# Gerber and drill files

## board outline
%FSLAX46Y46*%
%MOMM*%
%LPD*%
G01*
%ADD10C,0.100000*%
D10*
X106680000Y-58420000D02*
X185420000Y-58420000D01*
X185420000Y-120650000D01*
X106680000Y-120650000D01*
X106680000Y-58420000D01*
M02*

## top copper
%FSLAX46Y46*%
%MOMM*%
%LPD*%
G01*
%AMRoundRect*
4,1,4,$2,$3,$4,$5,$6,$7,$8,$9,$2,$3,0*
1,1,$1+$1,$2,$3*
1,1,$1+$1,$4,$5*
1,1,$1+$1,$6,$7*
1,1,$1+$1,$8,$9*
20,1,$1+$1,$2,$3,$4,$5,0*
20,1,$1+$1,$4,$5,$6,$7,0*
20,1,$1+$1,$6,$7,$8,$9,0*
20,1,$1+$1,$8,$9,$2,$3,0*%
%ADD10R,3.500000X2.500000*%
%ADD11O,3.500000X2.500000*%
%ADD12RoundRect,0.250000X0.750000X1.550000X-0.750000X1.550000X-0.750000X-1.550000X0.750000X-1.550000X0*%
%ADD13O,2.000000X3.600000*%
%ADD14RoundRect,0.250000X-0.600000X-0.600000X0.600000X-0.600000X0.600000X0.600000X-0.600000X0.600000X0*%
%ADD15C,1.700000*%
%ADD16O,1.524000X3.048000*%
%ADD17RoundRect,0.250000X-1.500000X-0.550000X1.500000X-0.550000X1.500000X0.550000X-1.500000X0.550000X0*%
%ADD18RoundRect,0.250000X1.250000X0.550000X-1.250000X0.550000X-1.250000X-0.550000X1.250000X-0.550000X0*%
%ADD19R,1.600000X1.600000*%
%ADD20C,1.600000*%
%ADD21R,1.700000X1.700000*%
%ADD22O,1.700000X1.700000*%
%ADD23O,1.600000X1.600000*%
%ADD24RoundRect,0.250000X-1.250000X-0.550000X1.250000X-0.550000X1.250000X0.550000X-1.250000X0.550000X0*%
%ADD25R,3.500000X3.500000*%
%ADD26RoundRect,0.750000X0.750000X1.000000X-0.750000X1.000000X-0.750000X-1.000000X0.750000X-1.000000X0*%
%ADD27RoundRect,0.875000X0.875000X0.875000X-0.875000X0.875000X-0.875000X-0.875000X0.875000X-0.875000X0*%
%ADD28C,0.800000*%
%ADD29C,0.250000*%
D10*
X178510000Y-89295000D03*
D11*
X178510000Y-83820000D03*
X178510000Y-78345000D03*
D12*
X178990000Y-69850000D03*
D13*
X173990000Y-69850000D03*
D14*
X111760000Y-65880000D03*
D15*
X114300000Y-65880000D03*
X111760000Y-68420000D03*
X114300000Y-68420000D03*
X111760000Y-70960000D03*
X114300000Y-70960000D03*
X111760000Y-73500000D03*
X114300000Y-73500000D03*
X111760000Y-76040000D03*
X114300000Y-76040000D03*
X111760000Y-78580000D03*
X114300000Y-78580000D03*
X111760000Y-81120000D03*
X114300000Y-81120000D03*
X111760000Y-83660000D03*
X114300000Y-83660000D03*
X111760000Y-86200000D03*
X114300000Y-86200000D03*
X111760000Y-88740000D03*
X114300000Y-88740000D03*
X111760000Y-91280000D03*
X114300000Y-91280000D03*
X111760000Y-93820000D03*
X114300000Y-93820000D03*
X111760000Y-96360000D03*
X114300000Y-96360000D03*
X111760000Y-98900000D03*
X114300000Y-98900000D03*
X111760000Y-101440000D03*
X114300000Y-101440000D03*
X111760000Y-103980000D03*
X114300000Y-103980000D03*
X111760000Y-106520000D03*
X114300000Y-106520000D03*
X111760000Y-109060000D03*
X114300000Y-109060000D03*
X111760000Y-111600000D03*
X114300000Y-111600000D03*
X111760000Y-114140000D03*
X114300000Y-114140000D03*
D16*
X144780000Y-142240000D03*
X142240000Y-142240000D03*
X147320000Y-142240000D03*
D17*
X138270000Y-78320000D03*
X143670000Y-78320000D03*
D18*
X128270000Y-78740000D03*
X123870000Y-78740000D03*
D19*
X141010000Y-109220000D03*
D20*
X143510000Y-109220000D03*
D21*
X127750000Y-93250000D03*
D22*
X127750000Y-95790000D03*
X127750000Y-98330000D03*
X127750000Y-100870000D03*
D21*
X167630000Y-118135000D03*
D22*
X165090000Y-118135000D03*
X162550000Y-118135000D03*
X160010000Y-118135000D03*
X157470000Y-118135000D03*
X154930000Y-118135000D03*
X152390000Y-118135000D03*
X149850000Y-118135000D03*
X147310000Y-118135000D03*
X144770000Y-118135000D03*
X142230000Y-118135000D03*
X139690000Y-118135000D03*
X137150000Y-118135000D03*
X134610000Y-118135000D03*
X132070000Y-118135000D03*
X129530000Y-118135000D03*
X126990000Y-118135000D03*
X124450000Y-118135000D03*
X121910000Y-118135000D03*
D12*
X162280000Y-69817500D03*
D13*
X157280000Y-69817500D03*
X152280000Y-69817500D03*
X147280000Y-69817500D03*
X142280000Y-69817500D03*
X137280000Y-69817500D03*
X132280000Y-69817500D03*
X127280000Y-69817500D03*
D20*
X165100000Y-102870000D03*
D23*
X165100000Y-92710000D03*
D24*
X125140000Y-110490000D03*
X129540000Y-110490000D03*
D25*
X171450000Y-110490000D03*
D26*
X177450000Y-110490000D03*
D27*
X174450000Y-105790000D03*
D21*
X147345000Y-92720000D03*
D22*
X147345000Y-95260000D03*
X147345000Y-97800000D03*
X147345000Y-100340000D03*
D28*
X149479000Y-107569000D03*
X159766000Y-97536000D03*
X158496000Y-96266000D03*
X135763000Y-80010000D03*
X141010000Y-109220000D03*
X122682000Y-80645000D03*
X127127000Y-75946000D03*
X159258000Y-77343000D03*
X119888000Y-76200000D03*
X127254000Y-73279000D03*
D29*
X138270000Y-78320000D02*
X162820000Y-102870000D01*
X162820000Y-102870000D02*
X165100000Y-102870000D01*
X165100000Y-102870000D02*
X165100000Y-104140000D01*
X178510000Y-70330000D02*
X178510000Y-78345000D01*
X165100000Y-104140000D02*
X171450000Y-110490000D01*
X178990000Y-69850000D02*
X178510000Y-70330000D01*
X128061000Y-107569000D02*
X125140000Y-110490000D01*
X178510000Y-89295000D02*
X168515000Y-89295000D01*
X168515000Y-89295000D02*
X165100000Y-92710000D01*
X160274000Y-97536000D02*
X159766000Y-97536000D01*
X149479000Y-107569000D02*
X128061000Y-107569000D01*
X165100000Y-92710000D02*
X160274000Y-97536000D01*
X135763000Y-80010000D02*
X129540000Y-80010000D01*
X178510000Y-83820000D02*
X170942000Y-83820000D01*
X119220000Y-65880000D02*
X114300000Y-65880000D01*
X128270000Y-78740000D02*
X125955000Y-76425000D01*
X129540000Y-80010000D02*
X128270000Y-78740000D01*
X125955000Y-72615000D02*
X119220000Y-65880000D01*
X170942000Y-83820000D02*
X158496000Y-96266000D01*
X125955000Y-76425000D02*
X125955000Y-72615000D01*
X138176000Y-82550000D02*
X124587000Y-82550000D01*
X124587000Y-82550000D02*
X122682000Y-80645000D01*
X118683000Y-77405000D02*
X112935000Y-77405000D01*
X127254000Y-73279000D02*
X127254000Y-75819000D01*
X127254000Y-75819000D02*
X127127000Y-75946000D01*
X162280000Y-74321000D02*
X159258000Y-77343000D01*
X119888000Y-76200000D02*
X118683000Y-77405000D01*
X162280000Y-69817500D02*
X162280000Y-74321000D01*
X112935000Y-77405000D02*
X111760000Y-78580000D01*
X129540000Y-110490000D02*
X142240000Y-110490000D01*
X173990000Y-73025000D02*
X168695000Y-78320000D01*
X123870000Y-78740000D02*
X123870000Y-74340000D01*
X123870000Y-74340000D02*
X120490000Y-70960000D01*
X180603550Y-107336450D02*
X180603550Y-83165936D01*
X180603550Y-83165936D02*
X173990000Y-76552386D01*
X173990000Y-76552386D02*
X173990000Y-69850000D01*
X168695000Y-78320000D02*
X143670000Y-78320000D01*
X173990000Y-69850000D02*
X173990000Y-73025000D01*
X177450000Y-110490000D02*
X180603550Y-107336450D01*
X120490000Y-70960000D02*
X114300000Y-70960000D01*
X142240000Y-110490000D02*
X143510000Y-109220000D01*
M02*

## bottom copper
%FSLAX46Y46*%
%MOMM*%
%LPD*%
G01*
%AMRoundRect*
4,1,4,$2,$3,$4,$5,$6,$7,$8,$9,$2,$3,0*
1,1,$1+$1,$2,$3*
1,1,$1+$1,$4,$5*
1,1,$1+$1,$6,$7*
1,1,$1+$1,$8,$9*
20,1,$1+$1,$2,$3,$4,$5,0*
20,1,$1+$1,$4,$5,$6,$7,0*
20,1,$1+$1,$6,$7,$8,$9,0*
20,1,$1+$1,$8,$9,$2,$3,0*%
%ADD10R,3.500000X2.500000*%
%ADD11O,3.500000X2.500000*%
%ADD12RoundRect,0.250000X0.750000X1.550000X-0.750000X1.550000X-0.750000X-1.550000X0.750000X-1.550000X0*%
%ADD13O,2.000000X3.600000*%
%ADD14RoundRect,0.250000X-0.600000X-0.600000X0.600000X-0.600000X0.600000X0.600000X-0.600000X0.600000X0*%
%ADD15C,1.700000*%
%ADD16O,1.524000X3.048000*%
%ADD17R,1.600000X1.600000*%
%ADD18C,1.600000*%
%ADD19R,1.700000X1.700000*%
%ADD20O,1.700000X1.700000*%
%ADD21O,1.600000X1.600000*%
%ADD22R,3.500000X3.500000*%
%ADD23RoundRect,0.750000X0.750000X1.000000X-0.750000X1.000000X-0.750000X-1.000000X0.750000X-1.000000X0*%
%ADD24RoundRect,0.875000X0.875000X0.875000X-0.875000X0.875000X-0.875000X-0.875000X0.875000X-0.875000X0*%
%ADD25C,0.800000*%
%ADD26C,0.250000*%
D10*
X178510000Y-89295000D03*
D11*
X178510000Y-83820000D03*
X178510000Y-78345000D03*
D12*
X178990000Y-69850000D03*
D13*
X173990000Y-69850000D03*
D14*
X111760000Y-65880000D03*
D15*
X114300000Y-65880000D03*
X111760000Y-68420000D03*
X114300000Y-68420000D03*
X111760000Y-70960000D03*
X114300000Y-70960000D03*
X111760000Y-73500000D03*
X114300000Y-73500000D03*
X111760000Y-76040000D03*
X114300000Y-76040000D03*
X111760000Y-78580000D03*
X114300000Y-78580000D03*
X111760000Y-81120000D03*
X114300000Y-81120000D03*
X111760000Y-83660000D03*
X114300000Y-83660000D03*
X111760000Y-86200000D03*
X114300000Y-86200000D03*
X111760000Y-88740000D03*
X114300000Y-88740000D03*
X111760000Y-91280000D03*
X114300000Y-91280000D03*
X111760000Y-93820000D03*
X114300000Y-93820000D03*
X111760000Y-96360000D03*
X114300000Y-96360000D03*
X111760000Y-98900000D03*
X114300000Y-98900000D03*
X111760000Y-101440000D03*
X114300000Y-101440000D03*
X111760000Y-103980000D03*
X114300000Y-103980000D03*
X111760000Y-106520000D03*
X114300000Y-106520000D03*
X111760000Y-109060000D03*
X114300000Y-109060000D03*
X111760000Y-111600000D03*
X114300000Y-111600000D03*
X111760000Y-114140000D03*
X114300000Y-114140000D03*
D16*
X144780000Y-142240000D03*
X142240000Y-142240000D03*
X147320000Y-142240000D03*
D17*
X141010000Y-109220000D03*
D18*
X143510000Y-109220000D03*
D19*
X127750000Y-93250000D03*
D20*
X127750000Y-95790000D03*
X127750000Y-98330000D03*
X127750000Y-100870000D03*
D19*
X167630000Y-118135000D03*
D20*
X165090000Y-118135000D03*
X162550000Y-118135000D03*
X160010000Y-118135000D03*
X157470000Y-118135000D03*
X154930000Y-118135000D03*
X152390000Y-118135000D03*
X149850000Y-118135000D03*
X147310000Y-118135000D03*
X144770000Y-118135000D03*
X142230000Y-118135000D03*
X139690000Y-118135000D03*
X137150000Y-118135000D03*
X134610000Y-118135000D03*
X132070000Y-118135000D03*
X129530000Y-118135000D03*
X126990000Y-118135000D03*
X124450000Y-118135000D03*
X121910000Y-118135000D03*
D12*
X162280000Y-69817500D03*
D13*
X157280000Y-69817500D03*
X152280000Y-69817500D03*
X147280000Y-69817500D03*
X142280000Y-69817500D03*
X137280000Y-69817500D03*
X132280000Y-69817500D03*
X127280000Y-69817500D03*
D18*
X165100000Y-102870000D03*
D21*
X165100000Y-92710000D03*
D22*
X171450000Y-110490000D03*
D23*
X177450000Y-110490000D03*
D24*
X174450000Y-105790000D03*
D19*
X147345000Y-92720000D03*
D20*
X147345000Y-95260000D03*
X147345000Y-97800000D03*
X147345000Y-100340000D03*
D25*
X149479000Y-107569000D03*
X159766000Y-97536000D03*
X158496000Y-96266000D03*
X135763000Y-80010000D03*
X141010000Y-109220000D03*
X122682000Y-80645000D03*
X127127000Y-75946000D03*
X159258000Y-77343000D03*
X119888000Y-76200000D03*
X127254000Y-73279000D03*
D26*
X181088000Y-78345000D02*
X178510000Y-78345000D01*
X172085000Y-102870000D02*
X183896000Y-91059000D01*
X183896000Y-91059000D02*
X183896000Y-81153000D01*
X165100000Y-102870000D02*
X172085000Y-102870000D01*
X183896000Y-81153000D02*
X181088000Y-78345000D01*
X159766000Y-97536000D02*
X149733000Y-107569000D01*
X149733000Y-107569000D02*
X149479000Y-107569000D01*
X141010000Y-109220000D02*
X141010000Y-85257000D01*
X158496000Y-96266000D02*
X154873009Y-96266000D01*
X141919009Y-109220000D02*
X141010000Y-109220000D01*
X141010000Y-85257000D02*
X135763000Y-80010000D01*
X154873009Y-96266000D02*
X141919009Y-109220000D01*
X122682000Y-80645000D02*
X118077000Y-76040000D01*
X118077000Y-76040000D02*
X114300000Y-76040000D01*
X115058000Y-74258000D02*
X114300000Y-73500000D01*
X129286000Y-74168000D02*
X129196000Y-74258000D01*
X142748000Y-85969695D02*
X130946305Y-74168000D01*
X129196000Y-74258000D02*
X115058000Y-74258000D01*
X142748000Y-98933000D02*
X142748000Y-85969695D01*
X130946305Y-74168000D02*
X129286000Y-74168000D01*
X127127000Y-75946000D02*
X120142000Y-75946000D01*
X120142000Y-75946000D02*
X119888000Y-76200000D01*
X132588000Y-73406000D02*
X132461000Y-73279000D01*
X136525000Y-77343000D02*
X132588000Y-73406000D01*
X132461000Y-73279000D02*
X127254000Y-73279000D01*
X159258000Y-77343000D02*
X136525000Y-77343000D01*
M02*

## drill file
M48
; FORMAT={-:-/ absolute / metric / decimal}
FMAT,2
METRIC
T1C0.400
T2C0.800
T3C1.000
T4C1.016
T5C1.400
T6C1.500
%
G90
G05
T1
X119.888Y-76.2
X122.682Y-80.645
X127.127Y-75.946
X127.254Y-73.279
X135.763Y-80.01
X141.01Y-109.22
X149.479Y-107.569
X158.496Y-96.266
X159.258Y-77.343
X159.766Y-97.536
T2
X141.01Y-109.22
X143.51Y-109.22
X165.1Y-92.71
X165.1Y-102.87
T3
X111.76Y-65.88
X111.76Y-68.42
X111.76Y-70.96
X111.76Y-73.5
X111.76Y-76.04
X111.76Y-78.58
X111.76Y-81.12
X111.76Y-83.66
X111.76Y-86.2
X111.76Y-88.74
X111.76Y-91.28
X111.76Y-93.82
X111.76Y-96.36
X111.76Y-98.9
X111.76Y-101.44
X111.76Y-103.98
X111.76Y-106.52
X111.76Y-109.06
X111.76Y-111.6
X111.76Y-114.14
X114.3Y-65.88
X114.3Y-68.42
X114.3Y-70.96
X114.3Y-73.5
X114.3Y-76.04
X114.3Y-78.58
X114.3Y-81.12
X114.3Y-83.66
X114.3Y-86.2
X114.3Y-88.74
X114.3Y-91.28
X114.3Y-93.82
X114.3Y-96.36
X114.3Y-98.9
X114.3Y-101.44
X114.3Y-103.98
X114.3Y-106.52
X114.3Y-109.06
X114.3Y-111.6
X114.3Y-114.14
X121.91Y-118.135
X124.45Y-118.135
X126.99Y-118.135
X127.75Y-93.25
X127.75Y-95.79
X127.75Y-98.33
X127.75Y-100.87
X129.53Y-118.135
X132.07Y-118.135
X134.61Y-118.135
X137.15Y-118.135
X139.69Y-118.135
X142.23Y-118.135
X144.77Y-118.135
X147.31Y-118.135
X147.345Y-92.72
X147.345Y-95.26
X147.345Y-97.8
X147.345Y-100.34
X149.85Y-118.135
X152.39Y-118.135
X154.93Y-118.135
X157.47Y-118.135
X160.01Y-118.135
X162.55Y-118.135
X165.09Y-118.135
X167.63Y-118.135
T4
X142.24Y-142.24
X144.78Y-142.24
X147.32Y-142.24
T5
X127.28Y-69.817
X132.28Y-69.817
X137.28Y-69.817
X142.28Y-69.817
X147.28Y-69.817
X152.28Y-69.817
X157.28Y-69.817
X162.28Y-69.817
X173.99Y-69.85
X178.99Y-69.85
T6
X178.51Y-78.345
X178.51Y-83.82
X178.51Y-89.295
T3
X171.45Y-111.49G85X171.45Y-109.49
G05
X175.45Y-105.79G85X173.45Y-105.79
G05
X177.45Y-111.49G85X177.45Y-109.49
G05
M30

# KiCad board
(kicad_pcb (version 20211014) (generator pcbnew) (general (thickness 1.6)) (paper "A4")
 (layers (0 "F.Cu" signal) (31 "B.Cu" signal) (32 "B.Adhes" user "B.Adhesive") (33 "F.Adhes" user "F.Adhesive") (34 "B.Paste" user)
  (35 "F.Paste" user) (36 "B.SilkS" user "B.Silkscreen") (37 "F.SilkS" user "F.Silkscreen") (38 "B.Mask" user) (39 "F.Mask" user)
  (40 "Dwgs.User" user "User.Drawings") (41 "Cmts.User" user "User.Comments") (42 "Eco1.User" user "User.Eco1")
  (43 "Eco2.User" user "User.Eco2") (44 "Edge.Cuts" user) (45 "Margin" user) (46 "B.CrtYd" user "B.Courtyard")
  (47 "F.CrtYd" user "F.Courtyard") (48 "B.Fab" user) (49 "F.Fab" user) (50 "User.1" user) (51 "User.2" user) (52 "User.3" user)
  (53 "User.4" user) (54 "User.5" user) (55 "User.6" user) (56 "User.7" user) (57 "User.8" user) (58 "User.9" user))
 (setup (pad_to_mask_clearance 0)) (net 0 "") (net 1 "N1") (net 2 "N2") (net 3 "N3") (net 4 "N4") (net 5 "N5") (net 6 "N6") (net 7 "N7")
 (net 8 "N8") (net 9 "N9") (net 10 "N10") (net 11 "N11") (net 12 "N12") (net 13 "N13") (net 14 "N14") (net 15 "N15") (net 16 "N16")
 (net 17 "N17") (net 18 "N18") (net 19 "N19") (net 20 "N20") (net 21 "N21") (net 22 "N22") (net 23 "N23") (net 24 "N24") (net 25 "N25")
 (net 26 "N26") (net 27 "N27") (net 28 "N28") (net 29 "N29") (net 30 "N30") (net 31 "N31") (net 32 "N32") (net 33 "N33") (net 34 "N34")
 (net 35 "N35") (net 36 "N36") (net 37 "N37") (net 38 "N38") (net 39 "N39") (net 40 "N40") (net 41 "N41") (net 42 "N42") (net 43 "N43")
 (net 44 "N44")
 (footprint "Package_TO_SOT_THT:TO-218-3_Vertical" (layer "F.Cu") (at 178.51 89.295 90)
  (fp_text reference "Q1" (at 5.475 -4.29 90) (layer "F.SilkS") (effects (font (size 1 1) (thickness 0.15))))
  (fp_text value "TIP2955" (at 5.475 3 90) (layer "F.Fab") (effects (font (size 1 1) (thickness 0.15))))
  (pad "1" thru_hole rect (at 0 0 90) (size 2.5 3.5) (drill 1.5) (layers *.Cu *.Mask) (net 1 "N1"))
  (pad "2" thru_hole oval (at 5.475 0 90) (size 2.5 3.5) (drill 1.5) (layers *.Cu *.Mask) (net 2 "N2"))
  (pad "3" thru_hole oval (at 10.95 0 90) (size 2.5 3.5) (drill 1.5) (layers *.Cu *.Mask) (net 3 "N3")))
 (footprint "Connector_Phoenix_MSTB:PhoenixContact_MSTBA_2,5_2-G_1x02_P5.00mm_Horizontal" (layer "F.Cu") (at 178.99 69.85 180)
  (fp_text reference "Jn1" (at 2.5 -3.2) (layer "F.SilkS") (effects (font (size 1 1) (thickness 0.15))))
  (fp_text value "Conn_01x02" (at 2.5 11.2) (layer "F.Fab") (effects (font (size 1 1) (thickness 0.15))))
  (pad "1" thru_hole roundrect (at 0 0 180) (size 2 3.6) (drill 1.4) (layers *.Cu *.Mask) (roundrect_rratio 0.125) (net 3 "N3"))
  (pad "2" thru_hole oval (at 5 0 180) (size 2 3.6) (drill 1.4) (layers *.Cu *.Mask) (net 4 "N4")))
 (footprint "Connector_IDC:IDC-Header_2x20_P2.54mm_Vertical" (layer "F.Cu") (at 111.76 65.88)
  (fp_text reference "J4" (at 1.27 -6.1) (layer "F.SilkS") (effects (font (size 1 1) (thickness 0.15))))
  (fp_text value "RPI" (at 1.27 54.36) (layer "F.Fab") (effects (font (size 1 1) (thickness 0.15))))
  (pad "1" thru_hole roundrect (at 0 0) (size 1.7 1.7) (drill 1) (layers *.Cu *.Mask) (roundrect_rratio 0.147059) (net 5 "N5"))
  (pad "2" thru_hole circle (at 2.54 0) (size 1.7 1.7) (drill 1) (layers *.Cu *.Mask) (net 2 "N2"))
  (pad "3" thru_hole circle (at 0 2.54) (size 1.7 1.7) (drill 1) (layers *.Cu *.Mask) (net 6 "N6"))
  (pad "4" thru_hole circle (at 2.54 2.54) (size 1.7 1.7) (drill 1) (layers *.Cu *.Mask) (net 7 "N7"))
  (pad "5" thru_hole circle (at 0 5.08) (size 1.7 1.7) (drill 1) (layers *.Cu *.Mask) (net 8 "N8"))
  (pad "6" thru_hole circle (at 2.54 5.08) (size 1.7 1.7) (drill 1) (layers *.Cu *.Mask) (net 4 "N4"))
  (pad "7" thru_hole circle (at 0 7.62) (size 1.7 1.7) (drill 1) (layers *.Cu *.Mask) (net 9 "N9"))
  (pad "8" thru_hole circle (at 2.54 7.62) (size 1.7 1.7) (drill 1) (layers *.Cu *.Mask) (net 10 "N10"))
  (pad "9" thru_hole circle (at 0 10.16) (size 1.7 1.7) (drill 1) (layers *.Cu *.Mask) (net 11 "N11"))
  (pad "10" thru_hole circle (at 2.54 10.16) (size 1.7 1.7) (drill 1) (layers *.Cu *.Mask) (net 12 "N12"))
  (pad "11" thru_hole circle (at 0 12.7) (size 1.7 1.7) (drill 1) (layers *.Cu *.Mask) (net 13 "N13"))
  (pad "12" thru_hole circle (at 2.54 12.7) (size 1.7 1.7) (drill 1) (layers *.Cu *.Mask) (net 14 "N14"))
  (pad "13" thru_hole circle (at 0 15.24) (size 1.7 1.7) (drill 1) (layers *.Cu *.Mask) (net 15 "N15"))
  (pad "14" thru_hole circle (at 2.54 15.24) (size 1.7 1.7) (drill 1) (layers *.Cu *.Mask) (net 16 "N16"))
  (pad "15" thru_hole circle (at 0 17.78) (size 1.7 1.7) (drill 1) (layers *.Cu *.Mask) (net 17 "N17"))
  (pad "16" thru_hole circle (at 2.54 17.78) (size 1.7 1.7) (drill 1) (layers *.Cu *.Mask) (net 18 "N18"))
  (pad "17" thru_hole circle (at 0 20.32) (size 1.7 1.7) (drill 1) (layers *.Cu *.Mask) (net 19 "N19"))
  (pad "18" thru_hole circle (at 2.54 20.32) (size 1.7 1.7) (drill 1) (layers *.Cu *.Mask) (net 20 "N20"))
  (pad "19" thru_hole circle (at 0 22.86) (size 1.7 1.7) (drill 1) (layers *.Cu *.Mask) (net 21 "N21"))
  (pad "20" thru_hole circle (at 2.54 22.86) (size 1.7 1.7) (drill 1) (layers *.Cu *.Mask) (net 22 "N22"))
  (pad "21" thru_hole circle (at 0 25.4) (size 1.7 1.7) (drill 1) (layers *.Cu *.Mask) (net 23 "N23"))
  (pad "22" thru_hole circle (at 2.54 25.4) (size 1.7 1.7) (drill 1) (layers *.Cu *.Mask) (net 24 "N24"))
  (pad "23" thru_hole circle (at 0 27.94) (size 1.7 1.7) (drill 1) (layers *.Cu *.Mask) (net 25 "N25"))
  (pad "24" thru_hole circle (at 2.54 27.94) (size 1.7 1.7) (drill 1) (layers *.Cu *.Mask) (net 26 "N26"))
  (pad "25" thru_hole circle (at 0 30.48) (size 1.7 1.7) (drill 1) (layers *.Cu *.Mask) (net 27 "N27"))
  (pad "26" thru_hole circle (at 2.54 30.48) (size 1.7 1.7) (drill 1) (layers *.Cu *.Mask) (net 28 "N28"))
  (pad "27" thru_hole circle (at 0 33.02) (size 1.7 1.7) (drill 1) (layers *.Cu *.Mask) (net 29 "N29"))
  (pad "28" thru_hole circle (at 2.54 33.02) (size 1.7 1.7) (drill 1) (layers *.Cu *.Mask) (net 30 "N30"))
  (pad "29" thru_hole circle (at 0 35.56) (size 1.7 1.7) (drill 1) (layers *.Cu *.Mask) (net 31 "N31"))
  (pad "30" thru_hole circle (at 2.54 35.56) (size 1.7 1.7) (drill 1) (layers *.Cu *.Mask) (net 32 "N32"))
  (pad "31" thru_hole circle (at 0 38.1) (size 1.7 1.7) (drill 1) (layers *.Cu *.Mask) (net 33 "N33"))
  (pad "32" thru_hole circle (at 2.54 38.1) (size 1.7 1.7) (drill 1) (layers *.Cu *.Mask) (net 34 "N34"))
  (pad "33" thru_hole circle (at 0 40.64) (size 1.7 1.7) (drill 1) (layers *.Cu *.Mask) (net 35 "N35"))
  (pad "34" thru_hole circle (at 2.54 40.64) (size 1.7 1.7) (drill 1) (layers *.Cu *.Mask) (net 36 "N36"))
  (pad "35" thru_hole circle (at 0 43.18) (size 1.7 1.7) (drill 1) (layers *.Cu *.Mask) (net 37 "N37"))
  (pad "36" thru_hole circle (at 2.54 43.18) (size 1.7 1.7) (drill 1) (layers *.Cu *.Mask) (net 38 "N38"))
  (pad "37" thru_hole circle (at 0 45.72) (size 1.7 1.7) (drill 1) (layers *.Cu *.Mask) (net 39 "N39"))
  (pad "38" thru_hole circle (at 2.54 45.72) (size 1.7 1.7) (drill 1) (layers *.Cu *.Mask) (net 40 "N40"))
  (pad "39" thru_hole circle (at 0 48.26) (size 1.7 1.7) (drill 1) (layers *.Cu *.Mask) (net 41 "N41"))
  (pad "40" thru_hole circle (at 2.54 48.26) (size 1.7 1.7) (drill 1) (layers *.Cu *.Mask) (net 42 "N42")))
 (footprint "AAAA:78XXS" (layer "F.Cu") (at 144.78 139.7)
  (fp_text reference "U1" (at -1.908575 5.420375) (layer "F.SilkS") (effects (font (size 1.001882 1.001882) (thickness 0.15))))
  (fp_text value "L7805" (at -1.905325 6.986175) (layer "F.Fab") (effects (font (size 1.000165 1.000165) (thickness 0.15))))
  (pad "GND" thru_hole oval locked (at 0 2.54) (size 1.524 3.048) (drill 1.016) (layers *.Cu *.Mask))
  (pad "IN" thru_hole oval locked (at -2.54 2.54) (size 1.524 3.048) (drill 1.016) (layers *.Cu *.Mask))
  (pad "OUT" thru_hole oval locked (at 2.54 2.54) (size 1.524 3.048) (drill 1.016) (layers *.Cu *.Mask)))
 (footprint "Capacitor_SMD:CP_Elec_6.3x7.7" (layer "F.Cu") (at 140.97 78.32)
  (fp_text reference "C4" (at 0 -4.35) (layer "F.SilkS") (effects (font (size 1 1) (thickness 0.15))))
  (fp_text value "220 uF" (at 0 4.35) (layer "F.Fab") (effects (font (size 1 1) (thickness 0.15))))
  (pad "1" smd roundrect (at -2.7 0) (size 3.5 1.6) (layers "F.Cu" "F.Paste" "F.Mask") (roundrect_rratio 0.15625) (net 3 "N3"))
  (pad "2" smd roundrect (at 2.7 0) (size 3.5 1.6) (layers "F.Cu" "F.Paste" "F.Mask") (roundrect_rratio 0.15625) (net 4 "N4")))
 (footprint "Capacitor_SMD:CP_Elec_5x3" (layer "F.Cu") (at 126.07 78.74 180)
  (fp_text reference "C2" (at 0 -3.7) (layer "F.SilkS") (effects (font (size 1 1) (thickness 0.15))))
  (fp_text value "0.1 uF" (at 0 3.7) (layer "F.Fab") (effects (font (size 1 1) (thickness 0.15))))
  (pad "1" smd roundrect (at -2.2 0 180) (size 3 1.6) (layers "F.Cu" "F.Paste" "F.Mask") (roundrect_rratio 0.15625) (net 2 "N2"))
  (pad "2" smd roundrect (at 2.2 0 180) (size 3 1.6) (layers "F.Cu" "F.Paste" "F.Mask") (roundrect_rratio 0.15625) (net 4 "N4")))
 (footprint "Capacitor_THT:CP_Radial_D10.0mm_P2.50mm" (layer "F.Cu") (at 141.01 109.22)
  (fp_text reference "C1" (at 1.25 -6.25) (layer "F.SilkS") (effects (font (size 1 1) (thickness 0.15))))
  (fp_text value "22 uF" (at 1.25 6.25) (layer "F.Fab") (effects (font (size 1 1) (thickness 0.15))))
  (pad "1" thru_hole rect (at 0 0) (size 1.6 1.6) (drill 0.8) (layers *.Cu *.Mask) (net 2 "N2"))
  (pad "2" thru_hole circle (at 2.5 0) (size 1.6 1.6) (drill 0.8) (layers *.Cu *.Mask) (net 4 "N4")))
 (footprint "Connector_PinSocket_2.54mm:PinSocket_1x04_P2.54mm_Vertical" (layer "F.Cu") (at 127.75 93.25)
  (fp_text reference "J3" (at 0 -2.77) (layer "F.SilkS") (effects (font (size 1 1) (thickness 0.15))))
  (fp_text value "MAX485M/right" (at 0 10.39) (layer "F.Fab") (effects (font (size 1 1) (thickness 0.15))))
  (pad "1" thru_hole rect (at 0 0) (size 1.7 1.7) (drill 1) (layers *.Cu *.Mask) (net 7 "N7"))
  (pad "2" thru_hole oval (at 0 2.54) (size 1.7 1.7) (drill 1) (layers *.Cu *.Mask) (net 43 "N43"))
  (pad "3" thru_hole oval (at 0 5.08) (size 1.7 1.7) (drill 1) (layers *.Cu *.Mask) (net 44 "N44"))
  (pad "4" thru_hole oval (at 0 7.62) (size 1.7 1.7) (drill 1) (layers *.Cu *.Mask) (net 16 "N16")))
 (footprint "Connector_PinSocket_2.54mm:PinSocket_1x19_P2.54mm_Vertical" (layer "F.Cu") (at 167.63 118.135 -90)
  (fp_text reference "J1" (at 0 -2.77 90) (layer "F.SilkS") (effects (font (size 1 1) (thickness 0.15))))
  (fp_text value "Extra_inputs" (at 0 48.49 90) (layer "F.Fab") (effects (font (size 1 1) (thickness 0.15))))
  (pad "1" thru_hole rect (at 0 0 270) (size 1.7 1.7) (drill 1) (layers *.Cu *.Mask) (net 5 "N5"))
  (pad "2" thru_hole oval (at 0 2.54 270) (size 1.7 1.7) (drill 1) (layers *.Cu *.Mask) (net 11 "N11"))
  (pad "3" thru_hole oval (at 0 5.08 270) (size 1.7 1.7) (drill 1) (layers *.Cu *.Mask) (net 19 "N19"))
  (pad "4" thru_hole oval (at 0 7.62 270) (size 1.7 1.7) (drill 1) (layers *.Cu *.Mask) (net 27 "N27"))
  (pad "5" thru_hole oval (at 0 10.16 270) (size 1.7 1.7) (drill 1) (layers *.Cu *.Mask) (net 6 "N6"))
  (pad "6" thru_hole oval (at 0 12.7 270) (size 1.7 1.7) (drill 1) (layers *.Cu *.Mask) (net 8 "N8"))
  (pad "7" thru_hole oval (at 0 15.24 270) (size 1.7 1.7) (drill 1) (layers *.Cu *.Mask) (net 9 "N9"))
  (pad "8" thru_hole oval (at 0 17.78 270) (size 1.7 1.7) (drill 1) (layers *.Cu *.Mask) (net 23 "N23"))
  (pad "9" thru_hole oval (at 0 20.32 270) (size 1.7 1.7) (drill 1) (layers *.Cu *.Mask) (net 21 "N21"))
  (pad "10" thru_hole oval (at 0 22.86 270) (size 1.7 1.7) (drill 1) (layers *.Cu *.Mask) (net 25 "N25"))
  (pad "11" thru_hole oval (at 0 25.4 270) (size 1.7 1.7) (drill 1) (layers *.Cu *.Mask) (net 35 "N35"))
  (pad "12" thru_hole oval (at 0 27.94 270) (size 1.7 1.7) (drill 1) (layers *.Cu *.Mask) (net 37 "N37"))
  (pad "13" thru_hole oval (at 0 30.48 270) (size 1.7 1.7) (drill 1) (layers *.Cu *.Mask) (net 14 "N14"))
  (pad "14" thru_hole oval (at 0 33.02 270) (size 1.7 1.7) (drill 1) (layers *.Cu *.Mask) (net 24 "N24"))
  (pad "15" thru_hole oval (at 0 35.56 270) (size 1.7 1.7) (drill 1) (layers *.Cu *.Mask) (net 26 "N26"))
  (pad "16" thru_hole oval (at 0 38.1 270) (size 1.7 1.7) (drill 1) (layers *.Cu *.Mask) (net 28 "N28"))
  (pad "17" thru_hole oval (at 0 40.64 270) (size 1.7 1.7) (drill 1) (layers *.Cu *.Mask) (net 38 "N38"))
  (pad "18" thru_hole oval (at 0 43.18 270) (size 1.7 1.7) (drill 1) (layers *.Cu *.Mask) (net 40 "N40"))
  (pad "19" thru_hole oval (at 0 45.72 270) (size 1.7 1.7) (drill 1) (layers *.Cu *.Mask) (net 42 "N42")))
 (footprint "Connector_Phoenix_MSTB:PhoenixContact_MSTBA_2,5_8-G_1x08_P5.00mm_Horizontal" (layer "F.Cu") (at 162.28 69.8175 180)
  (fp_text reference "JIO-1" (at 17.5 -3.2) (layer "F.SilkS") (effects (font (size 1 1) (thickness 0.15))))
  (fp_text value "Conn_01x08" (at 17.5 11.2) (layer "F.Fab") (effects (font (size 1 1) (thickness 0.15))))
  (pad "1" thru_hole roundrect (at 0 0 180) (size 2 3.6) (drill 1.4) (layers *.Cu *.Mask) (roundrect_rratio 0.125) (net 13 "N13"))
  (pad "2" thru_hole oval (at 5 0 180) (size 2 3.6) (drill 1.4) (layers *.Cu *.Mask) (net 15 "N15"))
  (pad "3" thru_hole oval (at 10 0 180) (size 2 3.6) (drill 1.4) (layers *.Cu *.Mask) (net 17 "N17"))
  (pad "4" thru_hole oval (at 15 0 180) (size 2 3.6) (drill 1.4) (layers *.Cu *.Mask) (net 31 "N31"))
  (pad "5" thru_hole oval (at 20 0 180) (size 2 3.6) (drill 1.4) (layers *.Cu *.Mask) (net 33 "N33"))
  (pad "6" thru_hole oval (at 25 0 180) (size 2 3.6) (drill 1.4) (layers *.Cu *.Mask) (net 39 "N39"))
  (pad "7" thru_hole oval (at 30 0 180) (size 2 3.6) (drill 1.4) (layers *.Cu *.Mask) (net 18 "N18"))
  (pad "8" thru_hole oval (at 35 0 180) (size 2 3.6) (drill 1.4) (layers *.Cu *.Mask) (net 20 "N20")))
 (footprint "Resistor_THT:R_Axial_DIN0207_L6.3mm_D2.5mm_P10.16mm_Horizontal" (layer "F.Cu") (at 165.1 102.87 90)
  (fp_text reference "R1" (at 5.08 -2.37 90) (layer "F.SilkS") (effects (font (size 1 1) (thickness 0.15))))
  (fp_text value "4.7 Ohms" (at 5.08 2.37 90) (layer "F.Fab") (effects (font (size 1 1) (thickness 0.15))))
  (pad "1" thru_hole circle (at 0 0 90) (size 1.6 1.6) (drill 0.8) (layers *.Cu *.Mask) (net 3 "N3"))
  (pad "2" thru_hole oval (at 10.16 0 90) (size 1.6 1.6) (drill 0.8) (layers *.Cu *.Mask) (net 1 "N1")))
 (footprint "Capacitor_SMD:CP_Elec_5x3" (layer "F.Cu") (at 127.34 110.49)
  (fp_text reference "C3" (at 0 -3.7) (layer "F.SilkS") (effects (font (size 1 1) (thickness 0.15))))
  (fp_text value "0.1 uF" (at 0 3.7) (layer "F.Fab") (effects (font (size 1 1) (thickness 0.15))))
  (pad "1" smd roundrect (at -2.2 0) (size 3 1.6) (layers "F.Cu" "F.Paste" "F.Mask") (roundrect_rratio 0.15625) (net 1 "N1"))
  (pad "2" smd roundrect (at 2.2 0) (size 3 1.6) (layers "F.Cu" "F.Paste" "F.Mask") (roundrect_rratio 0.15625) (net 4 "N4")))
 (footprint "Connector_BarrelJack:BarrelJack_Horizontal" (layer "F.Cu") (at 171.45 110.49 180)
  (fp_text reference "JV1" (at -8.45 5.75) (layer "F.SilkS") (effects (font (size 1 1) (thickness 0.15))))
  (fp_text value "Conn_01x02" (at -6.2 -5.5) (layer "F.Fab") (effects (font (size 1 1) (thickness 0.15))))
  (pad "1" thru_hole rect (at 0 0 180) (size 3.5 3.5) (drill oval 1 3) (layers *.Cu *.Mask) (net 3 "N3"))
  (pad "2" thru_hole roundrect (at -6 0 180) (size 3 3.5) (drill oval 1 3) (layers *.Cu *.Mask) (roundrect_rratio 0.25) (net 4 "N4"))
  (pad "3" thru_hole roundrect (at -3 4.7 180) (size 3.5 3.5) (drill oval 3 1) (layers *.Cu *.Mask) (roundrect_rratio 0.25)))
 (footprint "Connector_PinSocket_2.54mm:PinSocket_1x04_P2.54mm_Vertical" (layer "F.Cu") (at 147.345 92.72)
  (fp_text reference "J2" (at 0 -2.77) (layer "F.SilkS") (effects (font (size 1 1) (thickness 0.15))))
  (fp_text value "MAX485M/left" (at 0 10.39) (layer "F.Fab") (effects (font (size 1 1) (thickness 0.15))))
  (pad "1" thru_hole rect (at 0 0) (size 1.7 1.7) (drill 1) (layers *.Cu *.Mask) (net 12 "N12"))
  (pad "2" thru_hole oval (at 0 2.54) (size 1.7 1.7) (drill 1) (layers *.Cu *.Mask) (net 34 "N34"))
  (pad "3" thru_hole oval (at 0 5.08) (size 1.7 1.7) (drill 1) (layers *.Cu *.Mask) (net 34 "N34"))
  (pad "4" thru_hole oval (at 0 7.62) (size 1.7 1.7) (drill 1) (layers *.Cu *.Mask) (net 10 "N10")))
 (gr_rect (start 106.68 120.65) (end 185.42 58.42) (layer "Edge.Cuts") (width 0.1) (fill none))
 (segment (start 138.27 78.32) (end 162.82 102.87) (width 0.25) (layer "F.Cu") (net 3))
 (segment (start 162.82 102.87) (end 165.1 102.87) (width 0.25) (layer "F.Cu") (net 3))
 (segment (start 165.1 102.87) (end 165.1 104.14) (width 0.25) (layer "F.Cu") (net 3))
 (segment (start 178.51 70.33) (end 178.51 78.345) (width 0.25) (layer "F.Cu") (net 3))
 (segment (start 165.1 104.14) (end 171.45 110.49) (width 0.25) (layer "F.Cu") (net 3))
 (segment (start 178.99 69.85) (end 178.51 70.33) (width 0.25) (layer "F.Cu") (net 3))
 (segment (start 181.088 78.345) (end 178.51 78.345) (width 0.25) (layer "B.Cu") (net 3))
 (segment (start 172.085 102.87) (end 183.896 91.059) (width 0.25) (layer "B.Cu") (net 3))
 (segment (start 183.896 91.059) (end 183.896 81.153) (width 0.25) (layer "B.Cu") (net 3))
 (segment (start 165.1 102.87) (end 172.085 102.87) (width 0.25) (layer "B.Cu") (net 3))
 (segment (start 183.896 81.153) (end 181.088 78.345) (width 0.25) (layer "B.Cu") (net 3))
 (segment (start 128.061 107.569) (end 125.14 110.49) (width 0.25) (layer "F.Cu") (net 1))
 (segment (start 178.51 89.295) (end 168.515 89.295) (width 0.25) (layer "F.Cu") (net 1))
 (segment (start 168.515 89.295) (end 165.1 92.71) (width 0.25) (layer "F.Cu") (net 1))
 (segment (start 160.274 97.536) (end 159.766 97.536) (width 0.25) (layer "F.Cu") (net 1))
 (segment (start 149.479 107.569) (end 128.061 107.569) (width 0.25) (layer "F.Cu") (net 1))
 (segment (start 165.1 92.71) (end 160.274 97.536) (width 0.25) (layer "F.Cu") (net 1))
 (via (at 149.479 107.569) (size 0.8) (drill 0.4) (layers "F.Cu" "B.Cu") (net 1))
 (via (at 159.766 97.536) (size 0.8) (drill 0.4) (layers "F.Cu" "B.Cu") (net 1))
 (segment (start 159.766 97.536) (end 149.733 107.569) (width 0.25) (layer "B.Cu") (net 1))
 (segment (start 149.733 107.569) (end 149.479 107.569) (width 0.25) (layer "B.Cu") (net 1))
 (segment (start 135.763 80.01) (end 129.54 80.01) (width 0.25) (layer "F.Cu") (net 2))
 (segment (start 178.51 83.82) (end 170.942 83.82) (width 0.25) (layer "F.Cu") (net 2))
 (segment (start 119.22 65.88) (end 114.3 65.88) (width 0.25) (layer "F.Cu") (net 2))
 (segment (start 128.27 78.74) (end 125.955 76.425) (width 0.25) (layer "F.Cu") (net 2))
 (segment (start 129.54 80.01) (end 128.27 78.74) (width 0.25) (layer "F.Cu") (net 2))
 (segment (start 125.955 72.615) (end 119.22 65.88) (width 0.25) (layer "F.Cu") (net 2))
 (segment (start 170.942 83.82) (end 158.496 96.266) (width 0.25) (layer "F.Cu") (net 2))
 (segment (start 125.955 76.425) (end 125.955 72.615) (width 0.25) (layer "F.Cu") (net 2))
 (via (at 158.496 96.266) (size 0.8) (drill 0.4) (layers "F.Cu" "B.Cu") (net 2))
 (via (at 135.763 80.01) (size 0.8) (drill 0.4) (layers "F.Cu" "B.Cu") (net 2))
 (via (at 141.01 109.22) (size 0.8) (drill 0.4) (layers "F.Cu" "B.Cu") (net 2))
 (segment (start 141.01 109.22) (end 141.01 85.257) (width 0.25) (layer "B.Cu") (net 2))
 (segment (start 158.496 96.266) (end 154.873009 96.266) (width 0.25) (layer "B.Cu") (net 2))
 (segment (start 141.919009 109.22) (end 141.01 109.22) (width 0.25) (layer "B.Cu") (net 2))
 (segment (start 141.01 85.257) (end 135.763 80.01) (width 0.25) (layer "B.Cu") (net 2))
 (segment (start 154.873009 96.266) (end 141.919009 109.22) (width 0.25) (layer "B.Cu") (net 2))
 (segment (start 138.176 82.55) (end 124.587 82.55) (width 0.25) (layer "F.Cu") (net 12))
 (segment (start 124.587 82.55) (end 122.682 80.645) (width 0.25) (layer "F.Cu") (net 12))
 (via (at 122.682 80.645) (size 0.8) (drill 0.4) (layers "F.Cu" "B.Cu") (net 12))
 (segment (start 122.682 80.645) (end 118.077 76.04) (width 0.25) (layer "B.Cu") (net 12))
 (segment (start 118.077 76.04) (end 114.3 76.04) (width 0.25) (layer "B.Cu") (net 12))
 (segment (start 115.058 74.258) (end 114.3 73.5) (width 0.25) (layer "B.Cu") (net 10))
 (segment (start 129.286 74.168) (end 129.196 74.258) (width 0.25) (layer "B.Cu") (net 10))
 (segment (start 142.748 85.969695) (end 130.946305 74.168) (width 0.25) (layer "B.Cu") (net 10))
 (segment (start 129.196 74.258) (end 115.058 74.258) (width 0.25) (layer "B.Cu") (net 10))
 (segment (start 142.748 98.933) (end 142.748 85.969695) (width 0.25) (layer "B.Cu") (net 10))
 (segment (start 130.946305 74.168) (end 129.286 74.168) (width 0.25) (layer "B.Cu") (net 10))
 (segment (start 118.683 77.405) (end 112.935 77.405) (width 0.25) (layer "F.Cu") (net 13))
 (segment (start 127.254 73.279) (end 127.254 75.819) (width 0.25) (layer "F.Cu") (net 13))
 (segment (start 127.254 75.819) (end 127.127 75.946) (width 0.25) (layer "F.Cu") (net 13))
 (segment (start 162.28 74.321) (end 159.258 77.343) (width 0.25) (layer "F.Cu") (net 13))
 (segment (start 119.888 76.2) (end 118.683 77.405) (width 0.25) (layer "F.Cu") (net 13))
 (segment (start 162.28 69.8175) (end 162.28 74.321) (width 0.25) (layer "F.Cu") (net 13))
 (segment (start 112.935 77.405) (end 111.76 78.58) (width 0.25) (layer "F.Cu") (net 13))
 (via (at 127.127 75.946) (size 0.8) (drill 0.4) (layers "F.Cu" "B.Cu") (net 13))
 (via (at 159.258 77.343) (size 0.8) (drill 0.4) (layers "F.Cu" "B.Cu") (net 13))
 (via (at 119.888 76.2) (size 0.8) (drill 0.4) (layers "F.Cu" "B.Cu") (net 13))
 (via (at 127.254 73.279) (size 0.8) (drill 0.4) (layers "F.Cu" "B.Cu") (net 13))
 (segment (start 127.127 75.946) (end 120.142 75.946) (width 0.25) (layer "B.Cu") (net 13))
 (segment (start 120.142 75.946) (end 119.888 76.2) (width 0.25) (layer "B.Cu") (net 13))
 (segment (start 132.588 73.406) (end 132.461 73.279) (width 0.25) (layer "B.Cu") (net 13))
 (segment (start 136.525 77.343) (end 132.588 73.406) (width 0.25) (layer "B.Cu") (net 13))
 (segment (start 132.461 73.279) (end 127.254 73.279) (width 0.25) (layer "B.Cu") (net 13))
 (segment (start 159.258 77.343) (end 136.525 77.343) (width 0.25) (layer "B.Cu") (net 13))
 (segment (start 129.54 110.49) (end 142.24 110.49) (width 0.25) (layer "F.Cu") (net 4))
 (segment (start 173.99 73.025) (end 168.695 78.32) (width 0.25) (layer "F.Cu") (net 4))
 (segment (start 123.87 78.74) (end 123.87 74.34) (width 0.25) (layer "F.Cu") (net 4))
 (segment (start 123.87 74.34) (end 120.49 70.96) (width 0.25) (layer "F.Cu") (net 4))
 (segment (start 180.60355 107.33645) (end 180.60355 83.165936) (width 0.25) (layer "F.Cu") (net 4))
 (segment (start 180.60355 83.165936) (end 173.99 76.552386) (width 0.25) (layer "F.Cu") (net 4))
 (segment (start 173.99 76.552386) (end 173.99 69.85) (width 0.25) (layer "F.Cu") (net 4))
 (segment (start 168.695 78.32) (end 143.67 78.32) (width 0.25) (layer "F.Cu") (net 4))
 (segment (start 173.99 69.85) (end 173.99 73.025) (width 0.25) (layer "F.Cu") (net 4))
 (segment (start 177.45 110.49) (end 180.60355 107.33645) (width 0.25) (layer "F.Cu") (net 4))
 (segment (start 120.49 70.96) (end 114.3 70.96) (width 0.25) (layer "F.Cu") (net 4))
 (segment (start 142.24 110.49) (end 143.51 109.22) (width 0.25) (layer "F.Cu") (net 4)))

